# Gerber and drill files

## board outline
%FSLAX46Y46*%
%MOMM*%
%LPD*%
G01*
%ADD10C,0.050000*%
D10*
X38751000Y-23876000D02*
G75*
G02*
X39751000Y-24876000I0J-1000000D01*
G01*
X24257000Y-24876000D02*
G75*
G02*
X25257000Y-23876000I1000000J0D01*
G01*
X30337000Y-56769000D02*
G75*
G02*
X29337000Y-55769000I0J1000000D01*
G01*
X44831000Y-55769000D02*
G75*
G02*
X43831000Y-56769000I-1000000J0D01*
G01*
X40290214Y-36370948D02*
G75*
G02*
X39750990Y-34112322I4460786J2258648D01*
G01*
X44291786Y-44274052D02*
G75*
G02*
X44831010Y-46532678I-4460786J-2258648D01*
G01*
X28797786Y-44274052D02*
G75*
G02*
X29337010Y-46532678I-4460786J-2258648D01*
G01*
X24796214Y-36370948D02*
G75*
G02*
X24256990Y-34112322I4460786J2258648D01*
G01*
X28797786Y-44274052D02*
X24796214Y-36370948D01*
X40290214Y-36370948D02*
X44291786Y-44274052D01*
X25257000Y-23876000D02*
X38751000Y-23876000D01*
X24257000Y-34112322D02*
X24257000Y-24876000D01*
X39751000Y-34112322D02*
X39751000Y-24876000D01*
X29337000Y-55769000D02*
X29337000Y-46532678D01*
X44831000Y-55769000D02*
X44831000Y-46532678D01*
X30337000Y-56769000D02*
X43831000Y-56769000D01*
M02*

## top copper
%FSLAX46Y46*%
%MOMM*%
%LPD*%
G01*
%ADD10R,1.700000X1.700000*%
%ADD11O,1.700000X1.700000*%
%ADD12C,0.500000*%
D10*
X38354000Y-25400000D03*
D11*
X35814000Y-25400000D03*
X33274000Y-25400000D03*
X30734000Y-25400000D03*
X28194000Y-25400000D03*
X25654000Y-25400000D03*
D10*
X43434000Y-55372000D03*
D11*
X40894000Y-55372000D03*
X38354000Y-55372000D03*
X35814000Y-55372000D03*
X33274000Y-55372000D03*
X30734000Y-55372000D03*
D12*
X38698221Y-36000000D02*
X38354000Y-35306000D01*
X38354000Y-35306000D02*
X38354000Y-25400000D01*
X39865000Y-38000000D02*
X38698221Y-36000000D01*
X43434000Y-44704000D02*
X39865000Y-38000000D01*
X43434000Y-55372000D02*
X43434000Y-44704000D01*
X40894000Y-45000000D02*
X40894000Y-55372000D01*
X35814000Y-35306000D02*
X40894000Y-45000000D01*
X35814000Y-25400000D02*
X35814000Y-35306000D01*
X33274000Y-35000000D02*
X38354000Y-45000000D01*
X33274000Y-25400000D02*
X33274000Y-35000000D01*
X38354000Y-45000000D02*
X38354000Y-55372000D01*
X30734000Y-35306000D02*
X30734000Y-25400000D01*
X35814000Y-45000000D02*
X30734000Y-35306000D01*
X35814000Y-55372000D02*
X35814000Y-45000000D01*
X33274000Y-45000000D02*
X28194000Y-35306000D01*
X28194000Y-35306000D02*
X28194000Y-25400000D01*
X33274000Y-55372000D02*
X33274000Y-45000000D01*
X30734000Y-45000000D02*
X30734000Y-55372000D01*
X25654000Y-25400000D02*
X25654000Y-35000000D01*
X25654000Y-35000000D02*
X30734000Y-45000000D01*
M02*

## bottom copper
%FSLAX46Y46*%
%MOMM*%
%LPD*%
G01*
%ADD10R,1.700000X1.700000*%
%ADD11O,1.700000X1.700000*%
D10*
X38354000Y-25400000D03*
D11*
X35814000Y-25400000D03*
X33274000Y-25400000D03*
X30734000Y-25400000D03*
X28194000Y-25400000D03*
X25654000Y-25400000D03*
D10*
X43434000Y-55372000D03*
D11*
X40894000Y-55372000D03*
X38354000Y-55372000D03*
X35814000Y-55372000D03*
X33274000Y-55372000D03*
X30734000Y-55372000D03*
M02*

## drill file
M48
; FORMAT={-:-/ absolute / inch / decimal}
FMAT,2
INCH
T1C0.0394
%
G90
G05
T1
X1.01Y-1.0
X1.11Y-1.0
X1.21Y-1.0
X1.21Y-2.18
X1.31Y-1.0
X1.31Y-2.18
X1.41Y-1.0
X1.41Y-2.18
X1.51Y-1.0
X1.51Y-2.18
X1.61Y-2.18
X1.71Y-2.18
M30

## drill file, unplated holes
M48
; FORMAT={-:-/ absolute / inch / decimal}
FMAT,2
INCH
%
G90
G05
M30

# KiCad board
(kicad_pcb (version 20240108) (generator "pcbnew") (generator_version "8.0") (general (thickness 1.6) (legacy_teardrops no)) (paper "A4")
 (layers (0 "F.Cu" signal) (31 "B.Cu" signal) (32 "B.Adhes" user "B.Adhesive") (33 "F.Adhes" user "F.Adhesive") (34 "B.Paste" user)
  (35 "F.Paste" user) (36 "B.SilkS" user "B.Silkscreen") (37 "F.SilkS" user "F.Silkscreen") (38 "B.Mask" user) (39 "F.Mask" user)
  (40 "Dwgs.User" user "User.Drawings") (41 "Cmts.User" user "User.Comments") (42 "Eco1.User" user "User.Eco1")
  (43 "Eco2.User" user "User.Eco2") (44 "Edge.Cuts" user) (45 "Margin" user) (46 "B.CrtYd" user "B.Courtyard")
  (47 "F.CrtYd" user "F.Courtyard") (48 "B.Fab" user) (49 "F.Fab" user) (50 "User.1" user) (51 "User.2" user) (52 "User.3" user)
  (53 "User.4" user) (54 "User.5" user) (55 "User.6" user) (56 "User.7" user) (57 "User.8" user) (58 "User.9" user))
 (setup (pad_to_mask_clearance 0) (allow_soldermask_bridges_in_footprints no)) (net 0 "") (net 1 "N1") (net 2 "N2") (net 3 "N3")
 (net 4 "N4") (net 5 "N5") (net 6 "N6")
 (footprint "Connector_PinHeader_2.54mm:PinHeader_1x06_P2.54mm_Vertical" (layer "F.Cu") (at 38.354 25.4 -90)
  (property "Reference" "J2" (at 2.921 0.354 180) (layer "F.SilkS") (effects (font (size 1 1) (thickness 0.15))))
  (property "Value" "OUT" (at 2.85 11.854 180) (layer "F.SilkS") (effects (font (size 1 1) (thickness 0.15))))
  (pad "1" thru_hole rect (at 0 0 270) (size 1.7 1.7) (drill 1) (layers "*.Cu" "*.Mask") (remove_unused_layers no) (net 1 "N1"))
  (pad "2" thru_hole oval (at 0 2.54 270) (size 1.7 1.7) (drill 1) (layers "*.Cu" "*.Mask") (remove_unused_layers no) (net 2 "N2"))
  (pad "3" thru_hole oval (at 0 5.08 270) (size 1.7 1.7) (drill 1) (layers "*.Cu" "*.Mask") (remove_unused_layers no) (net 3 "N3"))
  (pad "4" thru_hole oval (at 0 7.62 270) (size 1.7 1.7) (drill 1) (layers "*.Cu" "*.Mask") (remove_unused_layers no) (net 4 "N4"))
  (pad "5" thru_hole oval (at 0 10.16 270) (size 1.7 1.7) (drill 1) (layers "*.Cu" "*.Mask") (remove_unused_layers no) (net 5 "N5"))
  (pad "6" thru_hole oval (at 0 12.7 270) (size 1.7 1.7) (drill 1) (layers "*.Cu" "*.Mask") (remove_unused_layers no) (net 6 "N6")))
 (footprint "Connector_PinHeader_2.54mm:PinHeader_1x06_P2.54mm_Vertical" (layer "F.Cu") (at 43.434 55.372 -90)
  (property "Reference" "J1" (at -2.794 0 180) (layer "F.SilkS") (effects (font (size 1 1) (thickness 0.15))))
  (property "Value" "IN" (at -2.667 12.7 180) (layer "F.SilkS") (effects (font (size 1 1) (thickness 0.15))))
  (pad "1" thru_hole rect (at 0 0 270) (size 1.7 1.7) (drill 1) (layers "*.Cu" "*.Mask") (remove_unused_layers no) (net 1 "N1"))
  (pad "2" thru_hole oval (at 0 2.54 270) (size 1.7 1.7) (drill 1) (layers "*.Cu" "*.Mask") (remove_unused_layers no) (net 2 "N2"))
  (pad "3" thru_hole oval (at 0 5.08 270) (size 1.7 1.7) (drill 1) (layers "*.Cu" "*.Mask") (remove_unused_layers no) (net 3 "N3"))
  (pad "4" thru_hole oval (at 0 7.62 270) (size 1.7 1.7) (drill 1) (layers "*.Cu" "*.Mask") (remove_unused_layers no) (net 4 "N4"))
  (pad "5" thru_hole oval (at 0 10.16 270) (size 1.7 1.7) (drill 1) (layers "*.Cu" "*.Mask") (remove_unused_layers no) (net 5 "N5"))
  (pad "6" thru_hole oval (at 0 12.7 270) (size 1.7 1.7) (drill 1) (layers "*.Cu" "*.Mask") (remove_unused_layers no) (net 6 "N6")))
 (gr_arc (start 44.291786 44.274052) (mid 44.694334 45.371628) (end 44.831 46.532678) (stroke (width 0.05) (type default))
  (layer "Edge.Cuts"))
 (gr_arc (start 24.796214 36.370948) (mid 24.393666 35.273372) (end 24.257 34.112322) (stroke (width 0.05) (type default))
  (layer "Edge.Cuts"))
 (gr_line (start 24.257 34.112322) (end 24.257 24.876) (stroke (width 0.05) (type default)) (layer "Edge.Cuts"))
 (gr_arc (start 38.751 23.876) (mid 39.458107 24.168893) (end 39.751 24.876) (stroke (width 0.05) (type default)) (layer "Edge.Cuts"))
 (gr_arc (start 24.257 24.876) (mid 24.549893 24.168893) (end 25.257 23.876) (stroke (width 0.05) (type default)) (layer "Edge.Cuts"))
 (gr_line (start 44.831 55.769) (end 44.831 46.532678) (stroke (width 0.05) (type default)) (layer "Edge.Cuts"))
 (gr_arc (start 30.337 56.769) (mid 29.629893 56.476107) (end 29.337 55.769) (stroke (width 0.05) (type default)) (layer "Edge.Cuts"))
 (gr_line (start 25.257 23.876) (end 38.751 23.876) (stroke (width 0.05) (type default)) (layer "Edge.Cuts"))
 (gr_line (start 28.797786 44.274052) (end 24.796214 36.370948) (stroke (width 0.05) (type default)) (layer "Edge.Cuts"))
 (gr_arc (start 28.797786 44.274052) (mid 29.200334 45.371628) (end 29.337 46.532678) (stroke (width 0.05) (type default))
  (layer "Edge.Cuts"))
 (gr_arc (start 44.831 55.769) (mid 44.538107 56.476107) (end 43.831 56.769) (stroke (width 0.05) (type default)) (layer "Edge.Cuts"))
 (gr_line (start 30.337 56.769) (end 43.831 56.769) (stroke (width 0.05) (type default)) (layer "Edge.Cuts"))
 (gr_arc (start 40.290214 36.370948) (mid 39.887666 35.273372) (end 39.751 34.112322) (stroke (width 0.05) (type default))
  (layer "Edge.Cuts"))
 (gr_line (start 29.337 55.769) (end 29.337 46.532678) (stroke (width 0.05) (type default)) (layer "Edge.Cuts"))
 (gr_line (start 39.751 34.112322) (end 39.751 24.876) (stroke (width 0.05) (type default)) (layer "Edge.Cuts"))
 (gr_line (start 40.290214 36.370948) (end 44.291786 44.274052) (stroke (width 0.05) (type default)) (layer "Edge.Cuts"))
 (segment (start 33.274 35) (end 38.354 45) (width 0.5) (layer "F.Cu") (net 3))
 (segment (start 38.354 45) (end 38.354 55.372) (width 0.5) (layer "F.Cu") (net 3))
 (segment (start 33.274 25.4) (end 33.274 35) (width 0.5) (layer "F.Cu") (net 3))
 (segment (start 28.194 35.306) (end 28.194 25.4) (width 0.5) (layer "F.Cu") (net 5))
 (segment (start 33.274 55.372) (end 33.274 45) (width 0.5) (layer "F.Cu") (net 5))
 (segment (start 33.274 45) (end 28.194 35.306) (width 0.5) (layer "F.Cu") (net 5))
 (segment (start 35.814 25.4) (end 35.814 35.306) (width 0.5) (layer "F.Cu") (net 2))
 (segment (start 35.814 35.306) (end 40.894 45) (width 0.5) (layer "F.Cu") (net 2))
 (segment (start 40.894 45) (end 40.894 55.372) (width 0.5) (layer "F.Cu") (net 2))
 (segment (start 35.814 45) (end 30.734 35.306) (width 0.5) (layer "F.Cu") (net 4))
 (segment (start 35.814 55.372) (end 35.814 45) (width 0.5) (layer "F.Cu") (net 4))
 (segment (start 30.734 35.306) (end 30.734 25.4) (width 0.5) (layer "F.Cu") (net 4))
 (segment (start 25.654 25.4) (end 25.654 35) (width 0.5) (layer "F.Cu") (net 6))
 (segment (start 25.654 35) (end 30.734 45) (width 0.5) (layer "F.Cu") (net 6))
 (segment (start 30.734 45) (end 30.734 55.372) (width 0.5) (layer "F.Cu") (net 6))
 (segment (start 39.865 38) (end 38.698221 36) (width 0.5) (layer "F.Cu") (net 1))
 (segment (start 38.698221 36) (end 38.354 35.306) (width 0.5) (layer "F.Cu") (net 1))
 (segment (start 38.354 35.306) (end 38.354 25.4) (width 0.5) (layer "F.Cu") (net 1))
 (segment (start 43.434 55.372) (end 43.434 44.704) (width 0.5) (layer "F.Cu") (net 1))
 (segment (start 43.434 44.704) (end 39.865 38) (width 0.5) (layer "F.Cu") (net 1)))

